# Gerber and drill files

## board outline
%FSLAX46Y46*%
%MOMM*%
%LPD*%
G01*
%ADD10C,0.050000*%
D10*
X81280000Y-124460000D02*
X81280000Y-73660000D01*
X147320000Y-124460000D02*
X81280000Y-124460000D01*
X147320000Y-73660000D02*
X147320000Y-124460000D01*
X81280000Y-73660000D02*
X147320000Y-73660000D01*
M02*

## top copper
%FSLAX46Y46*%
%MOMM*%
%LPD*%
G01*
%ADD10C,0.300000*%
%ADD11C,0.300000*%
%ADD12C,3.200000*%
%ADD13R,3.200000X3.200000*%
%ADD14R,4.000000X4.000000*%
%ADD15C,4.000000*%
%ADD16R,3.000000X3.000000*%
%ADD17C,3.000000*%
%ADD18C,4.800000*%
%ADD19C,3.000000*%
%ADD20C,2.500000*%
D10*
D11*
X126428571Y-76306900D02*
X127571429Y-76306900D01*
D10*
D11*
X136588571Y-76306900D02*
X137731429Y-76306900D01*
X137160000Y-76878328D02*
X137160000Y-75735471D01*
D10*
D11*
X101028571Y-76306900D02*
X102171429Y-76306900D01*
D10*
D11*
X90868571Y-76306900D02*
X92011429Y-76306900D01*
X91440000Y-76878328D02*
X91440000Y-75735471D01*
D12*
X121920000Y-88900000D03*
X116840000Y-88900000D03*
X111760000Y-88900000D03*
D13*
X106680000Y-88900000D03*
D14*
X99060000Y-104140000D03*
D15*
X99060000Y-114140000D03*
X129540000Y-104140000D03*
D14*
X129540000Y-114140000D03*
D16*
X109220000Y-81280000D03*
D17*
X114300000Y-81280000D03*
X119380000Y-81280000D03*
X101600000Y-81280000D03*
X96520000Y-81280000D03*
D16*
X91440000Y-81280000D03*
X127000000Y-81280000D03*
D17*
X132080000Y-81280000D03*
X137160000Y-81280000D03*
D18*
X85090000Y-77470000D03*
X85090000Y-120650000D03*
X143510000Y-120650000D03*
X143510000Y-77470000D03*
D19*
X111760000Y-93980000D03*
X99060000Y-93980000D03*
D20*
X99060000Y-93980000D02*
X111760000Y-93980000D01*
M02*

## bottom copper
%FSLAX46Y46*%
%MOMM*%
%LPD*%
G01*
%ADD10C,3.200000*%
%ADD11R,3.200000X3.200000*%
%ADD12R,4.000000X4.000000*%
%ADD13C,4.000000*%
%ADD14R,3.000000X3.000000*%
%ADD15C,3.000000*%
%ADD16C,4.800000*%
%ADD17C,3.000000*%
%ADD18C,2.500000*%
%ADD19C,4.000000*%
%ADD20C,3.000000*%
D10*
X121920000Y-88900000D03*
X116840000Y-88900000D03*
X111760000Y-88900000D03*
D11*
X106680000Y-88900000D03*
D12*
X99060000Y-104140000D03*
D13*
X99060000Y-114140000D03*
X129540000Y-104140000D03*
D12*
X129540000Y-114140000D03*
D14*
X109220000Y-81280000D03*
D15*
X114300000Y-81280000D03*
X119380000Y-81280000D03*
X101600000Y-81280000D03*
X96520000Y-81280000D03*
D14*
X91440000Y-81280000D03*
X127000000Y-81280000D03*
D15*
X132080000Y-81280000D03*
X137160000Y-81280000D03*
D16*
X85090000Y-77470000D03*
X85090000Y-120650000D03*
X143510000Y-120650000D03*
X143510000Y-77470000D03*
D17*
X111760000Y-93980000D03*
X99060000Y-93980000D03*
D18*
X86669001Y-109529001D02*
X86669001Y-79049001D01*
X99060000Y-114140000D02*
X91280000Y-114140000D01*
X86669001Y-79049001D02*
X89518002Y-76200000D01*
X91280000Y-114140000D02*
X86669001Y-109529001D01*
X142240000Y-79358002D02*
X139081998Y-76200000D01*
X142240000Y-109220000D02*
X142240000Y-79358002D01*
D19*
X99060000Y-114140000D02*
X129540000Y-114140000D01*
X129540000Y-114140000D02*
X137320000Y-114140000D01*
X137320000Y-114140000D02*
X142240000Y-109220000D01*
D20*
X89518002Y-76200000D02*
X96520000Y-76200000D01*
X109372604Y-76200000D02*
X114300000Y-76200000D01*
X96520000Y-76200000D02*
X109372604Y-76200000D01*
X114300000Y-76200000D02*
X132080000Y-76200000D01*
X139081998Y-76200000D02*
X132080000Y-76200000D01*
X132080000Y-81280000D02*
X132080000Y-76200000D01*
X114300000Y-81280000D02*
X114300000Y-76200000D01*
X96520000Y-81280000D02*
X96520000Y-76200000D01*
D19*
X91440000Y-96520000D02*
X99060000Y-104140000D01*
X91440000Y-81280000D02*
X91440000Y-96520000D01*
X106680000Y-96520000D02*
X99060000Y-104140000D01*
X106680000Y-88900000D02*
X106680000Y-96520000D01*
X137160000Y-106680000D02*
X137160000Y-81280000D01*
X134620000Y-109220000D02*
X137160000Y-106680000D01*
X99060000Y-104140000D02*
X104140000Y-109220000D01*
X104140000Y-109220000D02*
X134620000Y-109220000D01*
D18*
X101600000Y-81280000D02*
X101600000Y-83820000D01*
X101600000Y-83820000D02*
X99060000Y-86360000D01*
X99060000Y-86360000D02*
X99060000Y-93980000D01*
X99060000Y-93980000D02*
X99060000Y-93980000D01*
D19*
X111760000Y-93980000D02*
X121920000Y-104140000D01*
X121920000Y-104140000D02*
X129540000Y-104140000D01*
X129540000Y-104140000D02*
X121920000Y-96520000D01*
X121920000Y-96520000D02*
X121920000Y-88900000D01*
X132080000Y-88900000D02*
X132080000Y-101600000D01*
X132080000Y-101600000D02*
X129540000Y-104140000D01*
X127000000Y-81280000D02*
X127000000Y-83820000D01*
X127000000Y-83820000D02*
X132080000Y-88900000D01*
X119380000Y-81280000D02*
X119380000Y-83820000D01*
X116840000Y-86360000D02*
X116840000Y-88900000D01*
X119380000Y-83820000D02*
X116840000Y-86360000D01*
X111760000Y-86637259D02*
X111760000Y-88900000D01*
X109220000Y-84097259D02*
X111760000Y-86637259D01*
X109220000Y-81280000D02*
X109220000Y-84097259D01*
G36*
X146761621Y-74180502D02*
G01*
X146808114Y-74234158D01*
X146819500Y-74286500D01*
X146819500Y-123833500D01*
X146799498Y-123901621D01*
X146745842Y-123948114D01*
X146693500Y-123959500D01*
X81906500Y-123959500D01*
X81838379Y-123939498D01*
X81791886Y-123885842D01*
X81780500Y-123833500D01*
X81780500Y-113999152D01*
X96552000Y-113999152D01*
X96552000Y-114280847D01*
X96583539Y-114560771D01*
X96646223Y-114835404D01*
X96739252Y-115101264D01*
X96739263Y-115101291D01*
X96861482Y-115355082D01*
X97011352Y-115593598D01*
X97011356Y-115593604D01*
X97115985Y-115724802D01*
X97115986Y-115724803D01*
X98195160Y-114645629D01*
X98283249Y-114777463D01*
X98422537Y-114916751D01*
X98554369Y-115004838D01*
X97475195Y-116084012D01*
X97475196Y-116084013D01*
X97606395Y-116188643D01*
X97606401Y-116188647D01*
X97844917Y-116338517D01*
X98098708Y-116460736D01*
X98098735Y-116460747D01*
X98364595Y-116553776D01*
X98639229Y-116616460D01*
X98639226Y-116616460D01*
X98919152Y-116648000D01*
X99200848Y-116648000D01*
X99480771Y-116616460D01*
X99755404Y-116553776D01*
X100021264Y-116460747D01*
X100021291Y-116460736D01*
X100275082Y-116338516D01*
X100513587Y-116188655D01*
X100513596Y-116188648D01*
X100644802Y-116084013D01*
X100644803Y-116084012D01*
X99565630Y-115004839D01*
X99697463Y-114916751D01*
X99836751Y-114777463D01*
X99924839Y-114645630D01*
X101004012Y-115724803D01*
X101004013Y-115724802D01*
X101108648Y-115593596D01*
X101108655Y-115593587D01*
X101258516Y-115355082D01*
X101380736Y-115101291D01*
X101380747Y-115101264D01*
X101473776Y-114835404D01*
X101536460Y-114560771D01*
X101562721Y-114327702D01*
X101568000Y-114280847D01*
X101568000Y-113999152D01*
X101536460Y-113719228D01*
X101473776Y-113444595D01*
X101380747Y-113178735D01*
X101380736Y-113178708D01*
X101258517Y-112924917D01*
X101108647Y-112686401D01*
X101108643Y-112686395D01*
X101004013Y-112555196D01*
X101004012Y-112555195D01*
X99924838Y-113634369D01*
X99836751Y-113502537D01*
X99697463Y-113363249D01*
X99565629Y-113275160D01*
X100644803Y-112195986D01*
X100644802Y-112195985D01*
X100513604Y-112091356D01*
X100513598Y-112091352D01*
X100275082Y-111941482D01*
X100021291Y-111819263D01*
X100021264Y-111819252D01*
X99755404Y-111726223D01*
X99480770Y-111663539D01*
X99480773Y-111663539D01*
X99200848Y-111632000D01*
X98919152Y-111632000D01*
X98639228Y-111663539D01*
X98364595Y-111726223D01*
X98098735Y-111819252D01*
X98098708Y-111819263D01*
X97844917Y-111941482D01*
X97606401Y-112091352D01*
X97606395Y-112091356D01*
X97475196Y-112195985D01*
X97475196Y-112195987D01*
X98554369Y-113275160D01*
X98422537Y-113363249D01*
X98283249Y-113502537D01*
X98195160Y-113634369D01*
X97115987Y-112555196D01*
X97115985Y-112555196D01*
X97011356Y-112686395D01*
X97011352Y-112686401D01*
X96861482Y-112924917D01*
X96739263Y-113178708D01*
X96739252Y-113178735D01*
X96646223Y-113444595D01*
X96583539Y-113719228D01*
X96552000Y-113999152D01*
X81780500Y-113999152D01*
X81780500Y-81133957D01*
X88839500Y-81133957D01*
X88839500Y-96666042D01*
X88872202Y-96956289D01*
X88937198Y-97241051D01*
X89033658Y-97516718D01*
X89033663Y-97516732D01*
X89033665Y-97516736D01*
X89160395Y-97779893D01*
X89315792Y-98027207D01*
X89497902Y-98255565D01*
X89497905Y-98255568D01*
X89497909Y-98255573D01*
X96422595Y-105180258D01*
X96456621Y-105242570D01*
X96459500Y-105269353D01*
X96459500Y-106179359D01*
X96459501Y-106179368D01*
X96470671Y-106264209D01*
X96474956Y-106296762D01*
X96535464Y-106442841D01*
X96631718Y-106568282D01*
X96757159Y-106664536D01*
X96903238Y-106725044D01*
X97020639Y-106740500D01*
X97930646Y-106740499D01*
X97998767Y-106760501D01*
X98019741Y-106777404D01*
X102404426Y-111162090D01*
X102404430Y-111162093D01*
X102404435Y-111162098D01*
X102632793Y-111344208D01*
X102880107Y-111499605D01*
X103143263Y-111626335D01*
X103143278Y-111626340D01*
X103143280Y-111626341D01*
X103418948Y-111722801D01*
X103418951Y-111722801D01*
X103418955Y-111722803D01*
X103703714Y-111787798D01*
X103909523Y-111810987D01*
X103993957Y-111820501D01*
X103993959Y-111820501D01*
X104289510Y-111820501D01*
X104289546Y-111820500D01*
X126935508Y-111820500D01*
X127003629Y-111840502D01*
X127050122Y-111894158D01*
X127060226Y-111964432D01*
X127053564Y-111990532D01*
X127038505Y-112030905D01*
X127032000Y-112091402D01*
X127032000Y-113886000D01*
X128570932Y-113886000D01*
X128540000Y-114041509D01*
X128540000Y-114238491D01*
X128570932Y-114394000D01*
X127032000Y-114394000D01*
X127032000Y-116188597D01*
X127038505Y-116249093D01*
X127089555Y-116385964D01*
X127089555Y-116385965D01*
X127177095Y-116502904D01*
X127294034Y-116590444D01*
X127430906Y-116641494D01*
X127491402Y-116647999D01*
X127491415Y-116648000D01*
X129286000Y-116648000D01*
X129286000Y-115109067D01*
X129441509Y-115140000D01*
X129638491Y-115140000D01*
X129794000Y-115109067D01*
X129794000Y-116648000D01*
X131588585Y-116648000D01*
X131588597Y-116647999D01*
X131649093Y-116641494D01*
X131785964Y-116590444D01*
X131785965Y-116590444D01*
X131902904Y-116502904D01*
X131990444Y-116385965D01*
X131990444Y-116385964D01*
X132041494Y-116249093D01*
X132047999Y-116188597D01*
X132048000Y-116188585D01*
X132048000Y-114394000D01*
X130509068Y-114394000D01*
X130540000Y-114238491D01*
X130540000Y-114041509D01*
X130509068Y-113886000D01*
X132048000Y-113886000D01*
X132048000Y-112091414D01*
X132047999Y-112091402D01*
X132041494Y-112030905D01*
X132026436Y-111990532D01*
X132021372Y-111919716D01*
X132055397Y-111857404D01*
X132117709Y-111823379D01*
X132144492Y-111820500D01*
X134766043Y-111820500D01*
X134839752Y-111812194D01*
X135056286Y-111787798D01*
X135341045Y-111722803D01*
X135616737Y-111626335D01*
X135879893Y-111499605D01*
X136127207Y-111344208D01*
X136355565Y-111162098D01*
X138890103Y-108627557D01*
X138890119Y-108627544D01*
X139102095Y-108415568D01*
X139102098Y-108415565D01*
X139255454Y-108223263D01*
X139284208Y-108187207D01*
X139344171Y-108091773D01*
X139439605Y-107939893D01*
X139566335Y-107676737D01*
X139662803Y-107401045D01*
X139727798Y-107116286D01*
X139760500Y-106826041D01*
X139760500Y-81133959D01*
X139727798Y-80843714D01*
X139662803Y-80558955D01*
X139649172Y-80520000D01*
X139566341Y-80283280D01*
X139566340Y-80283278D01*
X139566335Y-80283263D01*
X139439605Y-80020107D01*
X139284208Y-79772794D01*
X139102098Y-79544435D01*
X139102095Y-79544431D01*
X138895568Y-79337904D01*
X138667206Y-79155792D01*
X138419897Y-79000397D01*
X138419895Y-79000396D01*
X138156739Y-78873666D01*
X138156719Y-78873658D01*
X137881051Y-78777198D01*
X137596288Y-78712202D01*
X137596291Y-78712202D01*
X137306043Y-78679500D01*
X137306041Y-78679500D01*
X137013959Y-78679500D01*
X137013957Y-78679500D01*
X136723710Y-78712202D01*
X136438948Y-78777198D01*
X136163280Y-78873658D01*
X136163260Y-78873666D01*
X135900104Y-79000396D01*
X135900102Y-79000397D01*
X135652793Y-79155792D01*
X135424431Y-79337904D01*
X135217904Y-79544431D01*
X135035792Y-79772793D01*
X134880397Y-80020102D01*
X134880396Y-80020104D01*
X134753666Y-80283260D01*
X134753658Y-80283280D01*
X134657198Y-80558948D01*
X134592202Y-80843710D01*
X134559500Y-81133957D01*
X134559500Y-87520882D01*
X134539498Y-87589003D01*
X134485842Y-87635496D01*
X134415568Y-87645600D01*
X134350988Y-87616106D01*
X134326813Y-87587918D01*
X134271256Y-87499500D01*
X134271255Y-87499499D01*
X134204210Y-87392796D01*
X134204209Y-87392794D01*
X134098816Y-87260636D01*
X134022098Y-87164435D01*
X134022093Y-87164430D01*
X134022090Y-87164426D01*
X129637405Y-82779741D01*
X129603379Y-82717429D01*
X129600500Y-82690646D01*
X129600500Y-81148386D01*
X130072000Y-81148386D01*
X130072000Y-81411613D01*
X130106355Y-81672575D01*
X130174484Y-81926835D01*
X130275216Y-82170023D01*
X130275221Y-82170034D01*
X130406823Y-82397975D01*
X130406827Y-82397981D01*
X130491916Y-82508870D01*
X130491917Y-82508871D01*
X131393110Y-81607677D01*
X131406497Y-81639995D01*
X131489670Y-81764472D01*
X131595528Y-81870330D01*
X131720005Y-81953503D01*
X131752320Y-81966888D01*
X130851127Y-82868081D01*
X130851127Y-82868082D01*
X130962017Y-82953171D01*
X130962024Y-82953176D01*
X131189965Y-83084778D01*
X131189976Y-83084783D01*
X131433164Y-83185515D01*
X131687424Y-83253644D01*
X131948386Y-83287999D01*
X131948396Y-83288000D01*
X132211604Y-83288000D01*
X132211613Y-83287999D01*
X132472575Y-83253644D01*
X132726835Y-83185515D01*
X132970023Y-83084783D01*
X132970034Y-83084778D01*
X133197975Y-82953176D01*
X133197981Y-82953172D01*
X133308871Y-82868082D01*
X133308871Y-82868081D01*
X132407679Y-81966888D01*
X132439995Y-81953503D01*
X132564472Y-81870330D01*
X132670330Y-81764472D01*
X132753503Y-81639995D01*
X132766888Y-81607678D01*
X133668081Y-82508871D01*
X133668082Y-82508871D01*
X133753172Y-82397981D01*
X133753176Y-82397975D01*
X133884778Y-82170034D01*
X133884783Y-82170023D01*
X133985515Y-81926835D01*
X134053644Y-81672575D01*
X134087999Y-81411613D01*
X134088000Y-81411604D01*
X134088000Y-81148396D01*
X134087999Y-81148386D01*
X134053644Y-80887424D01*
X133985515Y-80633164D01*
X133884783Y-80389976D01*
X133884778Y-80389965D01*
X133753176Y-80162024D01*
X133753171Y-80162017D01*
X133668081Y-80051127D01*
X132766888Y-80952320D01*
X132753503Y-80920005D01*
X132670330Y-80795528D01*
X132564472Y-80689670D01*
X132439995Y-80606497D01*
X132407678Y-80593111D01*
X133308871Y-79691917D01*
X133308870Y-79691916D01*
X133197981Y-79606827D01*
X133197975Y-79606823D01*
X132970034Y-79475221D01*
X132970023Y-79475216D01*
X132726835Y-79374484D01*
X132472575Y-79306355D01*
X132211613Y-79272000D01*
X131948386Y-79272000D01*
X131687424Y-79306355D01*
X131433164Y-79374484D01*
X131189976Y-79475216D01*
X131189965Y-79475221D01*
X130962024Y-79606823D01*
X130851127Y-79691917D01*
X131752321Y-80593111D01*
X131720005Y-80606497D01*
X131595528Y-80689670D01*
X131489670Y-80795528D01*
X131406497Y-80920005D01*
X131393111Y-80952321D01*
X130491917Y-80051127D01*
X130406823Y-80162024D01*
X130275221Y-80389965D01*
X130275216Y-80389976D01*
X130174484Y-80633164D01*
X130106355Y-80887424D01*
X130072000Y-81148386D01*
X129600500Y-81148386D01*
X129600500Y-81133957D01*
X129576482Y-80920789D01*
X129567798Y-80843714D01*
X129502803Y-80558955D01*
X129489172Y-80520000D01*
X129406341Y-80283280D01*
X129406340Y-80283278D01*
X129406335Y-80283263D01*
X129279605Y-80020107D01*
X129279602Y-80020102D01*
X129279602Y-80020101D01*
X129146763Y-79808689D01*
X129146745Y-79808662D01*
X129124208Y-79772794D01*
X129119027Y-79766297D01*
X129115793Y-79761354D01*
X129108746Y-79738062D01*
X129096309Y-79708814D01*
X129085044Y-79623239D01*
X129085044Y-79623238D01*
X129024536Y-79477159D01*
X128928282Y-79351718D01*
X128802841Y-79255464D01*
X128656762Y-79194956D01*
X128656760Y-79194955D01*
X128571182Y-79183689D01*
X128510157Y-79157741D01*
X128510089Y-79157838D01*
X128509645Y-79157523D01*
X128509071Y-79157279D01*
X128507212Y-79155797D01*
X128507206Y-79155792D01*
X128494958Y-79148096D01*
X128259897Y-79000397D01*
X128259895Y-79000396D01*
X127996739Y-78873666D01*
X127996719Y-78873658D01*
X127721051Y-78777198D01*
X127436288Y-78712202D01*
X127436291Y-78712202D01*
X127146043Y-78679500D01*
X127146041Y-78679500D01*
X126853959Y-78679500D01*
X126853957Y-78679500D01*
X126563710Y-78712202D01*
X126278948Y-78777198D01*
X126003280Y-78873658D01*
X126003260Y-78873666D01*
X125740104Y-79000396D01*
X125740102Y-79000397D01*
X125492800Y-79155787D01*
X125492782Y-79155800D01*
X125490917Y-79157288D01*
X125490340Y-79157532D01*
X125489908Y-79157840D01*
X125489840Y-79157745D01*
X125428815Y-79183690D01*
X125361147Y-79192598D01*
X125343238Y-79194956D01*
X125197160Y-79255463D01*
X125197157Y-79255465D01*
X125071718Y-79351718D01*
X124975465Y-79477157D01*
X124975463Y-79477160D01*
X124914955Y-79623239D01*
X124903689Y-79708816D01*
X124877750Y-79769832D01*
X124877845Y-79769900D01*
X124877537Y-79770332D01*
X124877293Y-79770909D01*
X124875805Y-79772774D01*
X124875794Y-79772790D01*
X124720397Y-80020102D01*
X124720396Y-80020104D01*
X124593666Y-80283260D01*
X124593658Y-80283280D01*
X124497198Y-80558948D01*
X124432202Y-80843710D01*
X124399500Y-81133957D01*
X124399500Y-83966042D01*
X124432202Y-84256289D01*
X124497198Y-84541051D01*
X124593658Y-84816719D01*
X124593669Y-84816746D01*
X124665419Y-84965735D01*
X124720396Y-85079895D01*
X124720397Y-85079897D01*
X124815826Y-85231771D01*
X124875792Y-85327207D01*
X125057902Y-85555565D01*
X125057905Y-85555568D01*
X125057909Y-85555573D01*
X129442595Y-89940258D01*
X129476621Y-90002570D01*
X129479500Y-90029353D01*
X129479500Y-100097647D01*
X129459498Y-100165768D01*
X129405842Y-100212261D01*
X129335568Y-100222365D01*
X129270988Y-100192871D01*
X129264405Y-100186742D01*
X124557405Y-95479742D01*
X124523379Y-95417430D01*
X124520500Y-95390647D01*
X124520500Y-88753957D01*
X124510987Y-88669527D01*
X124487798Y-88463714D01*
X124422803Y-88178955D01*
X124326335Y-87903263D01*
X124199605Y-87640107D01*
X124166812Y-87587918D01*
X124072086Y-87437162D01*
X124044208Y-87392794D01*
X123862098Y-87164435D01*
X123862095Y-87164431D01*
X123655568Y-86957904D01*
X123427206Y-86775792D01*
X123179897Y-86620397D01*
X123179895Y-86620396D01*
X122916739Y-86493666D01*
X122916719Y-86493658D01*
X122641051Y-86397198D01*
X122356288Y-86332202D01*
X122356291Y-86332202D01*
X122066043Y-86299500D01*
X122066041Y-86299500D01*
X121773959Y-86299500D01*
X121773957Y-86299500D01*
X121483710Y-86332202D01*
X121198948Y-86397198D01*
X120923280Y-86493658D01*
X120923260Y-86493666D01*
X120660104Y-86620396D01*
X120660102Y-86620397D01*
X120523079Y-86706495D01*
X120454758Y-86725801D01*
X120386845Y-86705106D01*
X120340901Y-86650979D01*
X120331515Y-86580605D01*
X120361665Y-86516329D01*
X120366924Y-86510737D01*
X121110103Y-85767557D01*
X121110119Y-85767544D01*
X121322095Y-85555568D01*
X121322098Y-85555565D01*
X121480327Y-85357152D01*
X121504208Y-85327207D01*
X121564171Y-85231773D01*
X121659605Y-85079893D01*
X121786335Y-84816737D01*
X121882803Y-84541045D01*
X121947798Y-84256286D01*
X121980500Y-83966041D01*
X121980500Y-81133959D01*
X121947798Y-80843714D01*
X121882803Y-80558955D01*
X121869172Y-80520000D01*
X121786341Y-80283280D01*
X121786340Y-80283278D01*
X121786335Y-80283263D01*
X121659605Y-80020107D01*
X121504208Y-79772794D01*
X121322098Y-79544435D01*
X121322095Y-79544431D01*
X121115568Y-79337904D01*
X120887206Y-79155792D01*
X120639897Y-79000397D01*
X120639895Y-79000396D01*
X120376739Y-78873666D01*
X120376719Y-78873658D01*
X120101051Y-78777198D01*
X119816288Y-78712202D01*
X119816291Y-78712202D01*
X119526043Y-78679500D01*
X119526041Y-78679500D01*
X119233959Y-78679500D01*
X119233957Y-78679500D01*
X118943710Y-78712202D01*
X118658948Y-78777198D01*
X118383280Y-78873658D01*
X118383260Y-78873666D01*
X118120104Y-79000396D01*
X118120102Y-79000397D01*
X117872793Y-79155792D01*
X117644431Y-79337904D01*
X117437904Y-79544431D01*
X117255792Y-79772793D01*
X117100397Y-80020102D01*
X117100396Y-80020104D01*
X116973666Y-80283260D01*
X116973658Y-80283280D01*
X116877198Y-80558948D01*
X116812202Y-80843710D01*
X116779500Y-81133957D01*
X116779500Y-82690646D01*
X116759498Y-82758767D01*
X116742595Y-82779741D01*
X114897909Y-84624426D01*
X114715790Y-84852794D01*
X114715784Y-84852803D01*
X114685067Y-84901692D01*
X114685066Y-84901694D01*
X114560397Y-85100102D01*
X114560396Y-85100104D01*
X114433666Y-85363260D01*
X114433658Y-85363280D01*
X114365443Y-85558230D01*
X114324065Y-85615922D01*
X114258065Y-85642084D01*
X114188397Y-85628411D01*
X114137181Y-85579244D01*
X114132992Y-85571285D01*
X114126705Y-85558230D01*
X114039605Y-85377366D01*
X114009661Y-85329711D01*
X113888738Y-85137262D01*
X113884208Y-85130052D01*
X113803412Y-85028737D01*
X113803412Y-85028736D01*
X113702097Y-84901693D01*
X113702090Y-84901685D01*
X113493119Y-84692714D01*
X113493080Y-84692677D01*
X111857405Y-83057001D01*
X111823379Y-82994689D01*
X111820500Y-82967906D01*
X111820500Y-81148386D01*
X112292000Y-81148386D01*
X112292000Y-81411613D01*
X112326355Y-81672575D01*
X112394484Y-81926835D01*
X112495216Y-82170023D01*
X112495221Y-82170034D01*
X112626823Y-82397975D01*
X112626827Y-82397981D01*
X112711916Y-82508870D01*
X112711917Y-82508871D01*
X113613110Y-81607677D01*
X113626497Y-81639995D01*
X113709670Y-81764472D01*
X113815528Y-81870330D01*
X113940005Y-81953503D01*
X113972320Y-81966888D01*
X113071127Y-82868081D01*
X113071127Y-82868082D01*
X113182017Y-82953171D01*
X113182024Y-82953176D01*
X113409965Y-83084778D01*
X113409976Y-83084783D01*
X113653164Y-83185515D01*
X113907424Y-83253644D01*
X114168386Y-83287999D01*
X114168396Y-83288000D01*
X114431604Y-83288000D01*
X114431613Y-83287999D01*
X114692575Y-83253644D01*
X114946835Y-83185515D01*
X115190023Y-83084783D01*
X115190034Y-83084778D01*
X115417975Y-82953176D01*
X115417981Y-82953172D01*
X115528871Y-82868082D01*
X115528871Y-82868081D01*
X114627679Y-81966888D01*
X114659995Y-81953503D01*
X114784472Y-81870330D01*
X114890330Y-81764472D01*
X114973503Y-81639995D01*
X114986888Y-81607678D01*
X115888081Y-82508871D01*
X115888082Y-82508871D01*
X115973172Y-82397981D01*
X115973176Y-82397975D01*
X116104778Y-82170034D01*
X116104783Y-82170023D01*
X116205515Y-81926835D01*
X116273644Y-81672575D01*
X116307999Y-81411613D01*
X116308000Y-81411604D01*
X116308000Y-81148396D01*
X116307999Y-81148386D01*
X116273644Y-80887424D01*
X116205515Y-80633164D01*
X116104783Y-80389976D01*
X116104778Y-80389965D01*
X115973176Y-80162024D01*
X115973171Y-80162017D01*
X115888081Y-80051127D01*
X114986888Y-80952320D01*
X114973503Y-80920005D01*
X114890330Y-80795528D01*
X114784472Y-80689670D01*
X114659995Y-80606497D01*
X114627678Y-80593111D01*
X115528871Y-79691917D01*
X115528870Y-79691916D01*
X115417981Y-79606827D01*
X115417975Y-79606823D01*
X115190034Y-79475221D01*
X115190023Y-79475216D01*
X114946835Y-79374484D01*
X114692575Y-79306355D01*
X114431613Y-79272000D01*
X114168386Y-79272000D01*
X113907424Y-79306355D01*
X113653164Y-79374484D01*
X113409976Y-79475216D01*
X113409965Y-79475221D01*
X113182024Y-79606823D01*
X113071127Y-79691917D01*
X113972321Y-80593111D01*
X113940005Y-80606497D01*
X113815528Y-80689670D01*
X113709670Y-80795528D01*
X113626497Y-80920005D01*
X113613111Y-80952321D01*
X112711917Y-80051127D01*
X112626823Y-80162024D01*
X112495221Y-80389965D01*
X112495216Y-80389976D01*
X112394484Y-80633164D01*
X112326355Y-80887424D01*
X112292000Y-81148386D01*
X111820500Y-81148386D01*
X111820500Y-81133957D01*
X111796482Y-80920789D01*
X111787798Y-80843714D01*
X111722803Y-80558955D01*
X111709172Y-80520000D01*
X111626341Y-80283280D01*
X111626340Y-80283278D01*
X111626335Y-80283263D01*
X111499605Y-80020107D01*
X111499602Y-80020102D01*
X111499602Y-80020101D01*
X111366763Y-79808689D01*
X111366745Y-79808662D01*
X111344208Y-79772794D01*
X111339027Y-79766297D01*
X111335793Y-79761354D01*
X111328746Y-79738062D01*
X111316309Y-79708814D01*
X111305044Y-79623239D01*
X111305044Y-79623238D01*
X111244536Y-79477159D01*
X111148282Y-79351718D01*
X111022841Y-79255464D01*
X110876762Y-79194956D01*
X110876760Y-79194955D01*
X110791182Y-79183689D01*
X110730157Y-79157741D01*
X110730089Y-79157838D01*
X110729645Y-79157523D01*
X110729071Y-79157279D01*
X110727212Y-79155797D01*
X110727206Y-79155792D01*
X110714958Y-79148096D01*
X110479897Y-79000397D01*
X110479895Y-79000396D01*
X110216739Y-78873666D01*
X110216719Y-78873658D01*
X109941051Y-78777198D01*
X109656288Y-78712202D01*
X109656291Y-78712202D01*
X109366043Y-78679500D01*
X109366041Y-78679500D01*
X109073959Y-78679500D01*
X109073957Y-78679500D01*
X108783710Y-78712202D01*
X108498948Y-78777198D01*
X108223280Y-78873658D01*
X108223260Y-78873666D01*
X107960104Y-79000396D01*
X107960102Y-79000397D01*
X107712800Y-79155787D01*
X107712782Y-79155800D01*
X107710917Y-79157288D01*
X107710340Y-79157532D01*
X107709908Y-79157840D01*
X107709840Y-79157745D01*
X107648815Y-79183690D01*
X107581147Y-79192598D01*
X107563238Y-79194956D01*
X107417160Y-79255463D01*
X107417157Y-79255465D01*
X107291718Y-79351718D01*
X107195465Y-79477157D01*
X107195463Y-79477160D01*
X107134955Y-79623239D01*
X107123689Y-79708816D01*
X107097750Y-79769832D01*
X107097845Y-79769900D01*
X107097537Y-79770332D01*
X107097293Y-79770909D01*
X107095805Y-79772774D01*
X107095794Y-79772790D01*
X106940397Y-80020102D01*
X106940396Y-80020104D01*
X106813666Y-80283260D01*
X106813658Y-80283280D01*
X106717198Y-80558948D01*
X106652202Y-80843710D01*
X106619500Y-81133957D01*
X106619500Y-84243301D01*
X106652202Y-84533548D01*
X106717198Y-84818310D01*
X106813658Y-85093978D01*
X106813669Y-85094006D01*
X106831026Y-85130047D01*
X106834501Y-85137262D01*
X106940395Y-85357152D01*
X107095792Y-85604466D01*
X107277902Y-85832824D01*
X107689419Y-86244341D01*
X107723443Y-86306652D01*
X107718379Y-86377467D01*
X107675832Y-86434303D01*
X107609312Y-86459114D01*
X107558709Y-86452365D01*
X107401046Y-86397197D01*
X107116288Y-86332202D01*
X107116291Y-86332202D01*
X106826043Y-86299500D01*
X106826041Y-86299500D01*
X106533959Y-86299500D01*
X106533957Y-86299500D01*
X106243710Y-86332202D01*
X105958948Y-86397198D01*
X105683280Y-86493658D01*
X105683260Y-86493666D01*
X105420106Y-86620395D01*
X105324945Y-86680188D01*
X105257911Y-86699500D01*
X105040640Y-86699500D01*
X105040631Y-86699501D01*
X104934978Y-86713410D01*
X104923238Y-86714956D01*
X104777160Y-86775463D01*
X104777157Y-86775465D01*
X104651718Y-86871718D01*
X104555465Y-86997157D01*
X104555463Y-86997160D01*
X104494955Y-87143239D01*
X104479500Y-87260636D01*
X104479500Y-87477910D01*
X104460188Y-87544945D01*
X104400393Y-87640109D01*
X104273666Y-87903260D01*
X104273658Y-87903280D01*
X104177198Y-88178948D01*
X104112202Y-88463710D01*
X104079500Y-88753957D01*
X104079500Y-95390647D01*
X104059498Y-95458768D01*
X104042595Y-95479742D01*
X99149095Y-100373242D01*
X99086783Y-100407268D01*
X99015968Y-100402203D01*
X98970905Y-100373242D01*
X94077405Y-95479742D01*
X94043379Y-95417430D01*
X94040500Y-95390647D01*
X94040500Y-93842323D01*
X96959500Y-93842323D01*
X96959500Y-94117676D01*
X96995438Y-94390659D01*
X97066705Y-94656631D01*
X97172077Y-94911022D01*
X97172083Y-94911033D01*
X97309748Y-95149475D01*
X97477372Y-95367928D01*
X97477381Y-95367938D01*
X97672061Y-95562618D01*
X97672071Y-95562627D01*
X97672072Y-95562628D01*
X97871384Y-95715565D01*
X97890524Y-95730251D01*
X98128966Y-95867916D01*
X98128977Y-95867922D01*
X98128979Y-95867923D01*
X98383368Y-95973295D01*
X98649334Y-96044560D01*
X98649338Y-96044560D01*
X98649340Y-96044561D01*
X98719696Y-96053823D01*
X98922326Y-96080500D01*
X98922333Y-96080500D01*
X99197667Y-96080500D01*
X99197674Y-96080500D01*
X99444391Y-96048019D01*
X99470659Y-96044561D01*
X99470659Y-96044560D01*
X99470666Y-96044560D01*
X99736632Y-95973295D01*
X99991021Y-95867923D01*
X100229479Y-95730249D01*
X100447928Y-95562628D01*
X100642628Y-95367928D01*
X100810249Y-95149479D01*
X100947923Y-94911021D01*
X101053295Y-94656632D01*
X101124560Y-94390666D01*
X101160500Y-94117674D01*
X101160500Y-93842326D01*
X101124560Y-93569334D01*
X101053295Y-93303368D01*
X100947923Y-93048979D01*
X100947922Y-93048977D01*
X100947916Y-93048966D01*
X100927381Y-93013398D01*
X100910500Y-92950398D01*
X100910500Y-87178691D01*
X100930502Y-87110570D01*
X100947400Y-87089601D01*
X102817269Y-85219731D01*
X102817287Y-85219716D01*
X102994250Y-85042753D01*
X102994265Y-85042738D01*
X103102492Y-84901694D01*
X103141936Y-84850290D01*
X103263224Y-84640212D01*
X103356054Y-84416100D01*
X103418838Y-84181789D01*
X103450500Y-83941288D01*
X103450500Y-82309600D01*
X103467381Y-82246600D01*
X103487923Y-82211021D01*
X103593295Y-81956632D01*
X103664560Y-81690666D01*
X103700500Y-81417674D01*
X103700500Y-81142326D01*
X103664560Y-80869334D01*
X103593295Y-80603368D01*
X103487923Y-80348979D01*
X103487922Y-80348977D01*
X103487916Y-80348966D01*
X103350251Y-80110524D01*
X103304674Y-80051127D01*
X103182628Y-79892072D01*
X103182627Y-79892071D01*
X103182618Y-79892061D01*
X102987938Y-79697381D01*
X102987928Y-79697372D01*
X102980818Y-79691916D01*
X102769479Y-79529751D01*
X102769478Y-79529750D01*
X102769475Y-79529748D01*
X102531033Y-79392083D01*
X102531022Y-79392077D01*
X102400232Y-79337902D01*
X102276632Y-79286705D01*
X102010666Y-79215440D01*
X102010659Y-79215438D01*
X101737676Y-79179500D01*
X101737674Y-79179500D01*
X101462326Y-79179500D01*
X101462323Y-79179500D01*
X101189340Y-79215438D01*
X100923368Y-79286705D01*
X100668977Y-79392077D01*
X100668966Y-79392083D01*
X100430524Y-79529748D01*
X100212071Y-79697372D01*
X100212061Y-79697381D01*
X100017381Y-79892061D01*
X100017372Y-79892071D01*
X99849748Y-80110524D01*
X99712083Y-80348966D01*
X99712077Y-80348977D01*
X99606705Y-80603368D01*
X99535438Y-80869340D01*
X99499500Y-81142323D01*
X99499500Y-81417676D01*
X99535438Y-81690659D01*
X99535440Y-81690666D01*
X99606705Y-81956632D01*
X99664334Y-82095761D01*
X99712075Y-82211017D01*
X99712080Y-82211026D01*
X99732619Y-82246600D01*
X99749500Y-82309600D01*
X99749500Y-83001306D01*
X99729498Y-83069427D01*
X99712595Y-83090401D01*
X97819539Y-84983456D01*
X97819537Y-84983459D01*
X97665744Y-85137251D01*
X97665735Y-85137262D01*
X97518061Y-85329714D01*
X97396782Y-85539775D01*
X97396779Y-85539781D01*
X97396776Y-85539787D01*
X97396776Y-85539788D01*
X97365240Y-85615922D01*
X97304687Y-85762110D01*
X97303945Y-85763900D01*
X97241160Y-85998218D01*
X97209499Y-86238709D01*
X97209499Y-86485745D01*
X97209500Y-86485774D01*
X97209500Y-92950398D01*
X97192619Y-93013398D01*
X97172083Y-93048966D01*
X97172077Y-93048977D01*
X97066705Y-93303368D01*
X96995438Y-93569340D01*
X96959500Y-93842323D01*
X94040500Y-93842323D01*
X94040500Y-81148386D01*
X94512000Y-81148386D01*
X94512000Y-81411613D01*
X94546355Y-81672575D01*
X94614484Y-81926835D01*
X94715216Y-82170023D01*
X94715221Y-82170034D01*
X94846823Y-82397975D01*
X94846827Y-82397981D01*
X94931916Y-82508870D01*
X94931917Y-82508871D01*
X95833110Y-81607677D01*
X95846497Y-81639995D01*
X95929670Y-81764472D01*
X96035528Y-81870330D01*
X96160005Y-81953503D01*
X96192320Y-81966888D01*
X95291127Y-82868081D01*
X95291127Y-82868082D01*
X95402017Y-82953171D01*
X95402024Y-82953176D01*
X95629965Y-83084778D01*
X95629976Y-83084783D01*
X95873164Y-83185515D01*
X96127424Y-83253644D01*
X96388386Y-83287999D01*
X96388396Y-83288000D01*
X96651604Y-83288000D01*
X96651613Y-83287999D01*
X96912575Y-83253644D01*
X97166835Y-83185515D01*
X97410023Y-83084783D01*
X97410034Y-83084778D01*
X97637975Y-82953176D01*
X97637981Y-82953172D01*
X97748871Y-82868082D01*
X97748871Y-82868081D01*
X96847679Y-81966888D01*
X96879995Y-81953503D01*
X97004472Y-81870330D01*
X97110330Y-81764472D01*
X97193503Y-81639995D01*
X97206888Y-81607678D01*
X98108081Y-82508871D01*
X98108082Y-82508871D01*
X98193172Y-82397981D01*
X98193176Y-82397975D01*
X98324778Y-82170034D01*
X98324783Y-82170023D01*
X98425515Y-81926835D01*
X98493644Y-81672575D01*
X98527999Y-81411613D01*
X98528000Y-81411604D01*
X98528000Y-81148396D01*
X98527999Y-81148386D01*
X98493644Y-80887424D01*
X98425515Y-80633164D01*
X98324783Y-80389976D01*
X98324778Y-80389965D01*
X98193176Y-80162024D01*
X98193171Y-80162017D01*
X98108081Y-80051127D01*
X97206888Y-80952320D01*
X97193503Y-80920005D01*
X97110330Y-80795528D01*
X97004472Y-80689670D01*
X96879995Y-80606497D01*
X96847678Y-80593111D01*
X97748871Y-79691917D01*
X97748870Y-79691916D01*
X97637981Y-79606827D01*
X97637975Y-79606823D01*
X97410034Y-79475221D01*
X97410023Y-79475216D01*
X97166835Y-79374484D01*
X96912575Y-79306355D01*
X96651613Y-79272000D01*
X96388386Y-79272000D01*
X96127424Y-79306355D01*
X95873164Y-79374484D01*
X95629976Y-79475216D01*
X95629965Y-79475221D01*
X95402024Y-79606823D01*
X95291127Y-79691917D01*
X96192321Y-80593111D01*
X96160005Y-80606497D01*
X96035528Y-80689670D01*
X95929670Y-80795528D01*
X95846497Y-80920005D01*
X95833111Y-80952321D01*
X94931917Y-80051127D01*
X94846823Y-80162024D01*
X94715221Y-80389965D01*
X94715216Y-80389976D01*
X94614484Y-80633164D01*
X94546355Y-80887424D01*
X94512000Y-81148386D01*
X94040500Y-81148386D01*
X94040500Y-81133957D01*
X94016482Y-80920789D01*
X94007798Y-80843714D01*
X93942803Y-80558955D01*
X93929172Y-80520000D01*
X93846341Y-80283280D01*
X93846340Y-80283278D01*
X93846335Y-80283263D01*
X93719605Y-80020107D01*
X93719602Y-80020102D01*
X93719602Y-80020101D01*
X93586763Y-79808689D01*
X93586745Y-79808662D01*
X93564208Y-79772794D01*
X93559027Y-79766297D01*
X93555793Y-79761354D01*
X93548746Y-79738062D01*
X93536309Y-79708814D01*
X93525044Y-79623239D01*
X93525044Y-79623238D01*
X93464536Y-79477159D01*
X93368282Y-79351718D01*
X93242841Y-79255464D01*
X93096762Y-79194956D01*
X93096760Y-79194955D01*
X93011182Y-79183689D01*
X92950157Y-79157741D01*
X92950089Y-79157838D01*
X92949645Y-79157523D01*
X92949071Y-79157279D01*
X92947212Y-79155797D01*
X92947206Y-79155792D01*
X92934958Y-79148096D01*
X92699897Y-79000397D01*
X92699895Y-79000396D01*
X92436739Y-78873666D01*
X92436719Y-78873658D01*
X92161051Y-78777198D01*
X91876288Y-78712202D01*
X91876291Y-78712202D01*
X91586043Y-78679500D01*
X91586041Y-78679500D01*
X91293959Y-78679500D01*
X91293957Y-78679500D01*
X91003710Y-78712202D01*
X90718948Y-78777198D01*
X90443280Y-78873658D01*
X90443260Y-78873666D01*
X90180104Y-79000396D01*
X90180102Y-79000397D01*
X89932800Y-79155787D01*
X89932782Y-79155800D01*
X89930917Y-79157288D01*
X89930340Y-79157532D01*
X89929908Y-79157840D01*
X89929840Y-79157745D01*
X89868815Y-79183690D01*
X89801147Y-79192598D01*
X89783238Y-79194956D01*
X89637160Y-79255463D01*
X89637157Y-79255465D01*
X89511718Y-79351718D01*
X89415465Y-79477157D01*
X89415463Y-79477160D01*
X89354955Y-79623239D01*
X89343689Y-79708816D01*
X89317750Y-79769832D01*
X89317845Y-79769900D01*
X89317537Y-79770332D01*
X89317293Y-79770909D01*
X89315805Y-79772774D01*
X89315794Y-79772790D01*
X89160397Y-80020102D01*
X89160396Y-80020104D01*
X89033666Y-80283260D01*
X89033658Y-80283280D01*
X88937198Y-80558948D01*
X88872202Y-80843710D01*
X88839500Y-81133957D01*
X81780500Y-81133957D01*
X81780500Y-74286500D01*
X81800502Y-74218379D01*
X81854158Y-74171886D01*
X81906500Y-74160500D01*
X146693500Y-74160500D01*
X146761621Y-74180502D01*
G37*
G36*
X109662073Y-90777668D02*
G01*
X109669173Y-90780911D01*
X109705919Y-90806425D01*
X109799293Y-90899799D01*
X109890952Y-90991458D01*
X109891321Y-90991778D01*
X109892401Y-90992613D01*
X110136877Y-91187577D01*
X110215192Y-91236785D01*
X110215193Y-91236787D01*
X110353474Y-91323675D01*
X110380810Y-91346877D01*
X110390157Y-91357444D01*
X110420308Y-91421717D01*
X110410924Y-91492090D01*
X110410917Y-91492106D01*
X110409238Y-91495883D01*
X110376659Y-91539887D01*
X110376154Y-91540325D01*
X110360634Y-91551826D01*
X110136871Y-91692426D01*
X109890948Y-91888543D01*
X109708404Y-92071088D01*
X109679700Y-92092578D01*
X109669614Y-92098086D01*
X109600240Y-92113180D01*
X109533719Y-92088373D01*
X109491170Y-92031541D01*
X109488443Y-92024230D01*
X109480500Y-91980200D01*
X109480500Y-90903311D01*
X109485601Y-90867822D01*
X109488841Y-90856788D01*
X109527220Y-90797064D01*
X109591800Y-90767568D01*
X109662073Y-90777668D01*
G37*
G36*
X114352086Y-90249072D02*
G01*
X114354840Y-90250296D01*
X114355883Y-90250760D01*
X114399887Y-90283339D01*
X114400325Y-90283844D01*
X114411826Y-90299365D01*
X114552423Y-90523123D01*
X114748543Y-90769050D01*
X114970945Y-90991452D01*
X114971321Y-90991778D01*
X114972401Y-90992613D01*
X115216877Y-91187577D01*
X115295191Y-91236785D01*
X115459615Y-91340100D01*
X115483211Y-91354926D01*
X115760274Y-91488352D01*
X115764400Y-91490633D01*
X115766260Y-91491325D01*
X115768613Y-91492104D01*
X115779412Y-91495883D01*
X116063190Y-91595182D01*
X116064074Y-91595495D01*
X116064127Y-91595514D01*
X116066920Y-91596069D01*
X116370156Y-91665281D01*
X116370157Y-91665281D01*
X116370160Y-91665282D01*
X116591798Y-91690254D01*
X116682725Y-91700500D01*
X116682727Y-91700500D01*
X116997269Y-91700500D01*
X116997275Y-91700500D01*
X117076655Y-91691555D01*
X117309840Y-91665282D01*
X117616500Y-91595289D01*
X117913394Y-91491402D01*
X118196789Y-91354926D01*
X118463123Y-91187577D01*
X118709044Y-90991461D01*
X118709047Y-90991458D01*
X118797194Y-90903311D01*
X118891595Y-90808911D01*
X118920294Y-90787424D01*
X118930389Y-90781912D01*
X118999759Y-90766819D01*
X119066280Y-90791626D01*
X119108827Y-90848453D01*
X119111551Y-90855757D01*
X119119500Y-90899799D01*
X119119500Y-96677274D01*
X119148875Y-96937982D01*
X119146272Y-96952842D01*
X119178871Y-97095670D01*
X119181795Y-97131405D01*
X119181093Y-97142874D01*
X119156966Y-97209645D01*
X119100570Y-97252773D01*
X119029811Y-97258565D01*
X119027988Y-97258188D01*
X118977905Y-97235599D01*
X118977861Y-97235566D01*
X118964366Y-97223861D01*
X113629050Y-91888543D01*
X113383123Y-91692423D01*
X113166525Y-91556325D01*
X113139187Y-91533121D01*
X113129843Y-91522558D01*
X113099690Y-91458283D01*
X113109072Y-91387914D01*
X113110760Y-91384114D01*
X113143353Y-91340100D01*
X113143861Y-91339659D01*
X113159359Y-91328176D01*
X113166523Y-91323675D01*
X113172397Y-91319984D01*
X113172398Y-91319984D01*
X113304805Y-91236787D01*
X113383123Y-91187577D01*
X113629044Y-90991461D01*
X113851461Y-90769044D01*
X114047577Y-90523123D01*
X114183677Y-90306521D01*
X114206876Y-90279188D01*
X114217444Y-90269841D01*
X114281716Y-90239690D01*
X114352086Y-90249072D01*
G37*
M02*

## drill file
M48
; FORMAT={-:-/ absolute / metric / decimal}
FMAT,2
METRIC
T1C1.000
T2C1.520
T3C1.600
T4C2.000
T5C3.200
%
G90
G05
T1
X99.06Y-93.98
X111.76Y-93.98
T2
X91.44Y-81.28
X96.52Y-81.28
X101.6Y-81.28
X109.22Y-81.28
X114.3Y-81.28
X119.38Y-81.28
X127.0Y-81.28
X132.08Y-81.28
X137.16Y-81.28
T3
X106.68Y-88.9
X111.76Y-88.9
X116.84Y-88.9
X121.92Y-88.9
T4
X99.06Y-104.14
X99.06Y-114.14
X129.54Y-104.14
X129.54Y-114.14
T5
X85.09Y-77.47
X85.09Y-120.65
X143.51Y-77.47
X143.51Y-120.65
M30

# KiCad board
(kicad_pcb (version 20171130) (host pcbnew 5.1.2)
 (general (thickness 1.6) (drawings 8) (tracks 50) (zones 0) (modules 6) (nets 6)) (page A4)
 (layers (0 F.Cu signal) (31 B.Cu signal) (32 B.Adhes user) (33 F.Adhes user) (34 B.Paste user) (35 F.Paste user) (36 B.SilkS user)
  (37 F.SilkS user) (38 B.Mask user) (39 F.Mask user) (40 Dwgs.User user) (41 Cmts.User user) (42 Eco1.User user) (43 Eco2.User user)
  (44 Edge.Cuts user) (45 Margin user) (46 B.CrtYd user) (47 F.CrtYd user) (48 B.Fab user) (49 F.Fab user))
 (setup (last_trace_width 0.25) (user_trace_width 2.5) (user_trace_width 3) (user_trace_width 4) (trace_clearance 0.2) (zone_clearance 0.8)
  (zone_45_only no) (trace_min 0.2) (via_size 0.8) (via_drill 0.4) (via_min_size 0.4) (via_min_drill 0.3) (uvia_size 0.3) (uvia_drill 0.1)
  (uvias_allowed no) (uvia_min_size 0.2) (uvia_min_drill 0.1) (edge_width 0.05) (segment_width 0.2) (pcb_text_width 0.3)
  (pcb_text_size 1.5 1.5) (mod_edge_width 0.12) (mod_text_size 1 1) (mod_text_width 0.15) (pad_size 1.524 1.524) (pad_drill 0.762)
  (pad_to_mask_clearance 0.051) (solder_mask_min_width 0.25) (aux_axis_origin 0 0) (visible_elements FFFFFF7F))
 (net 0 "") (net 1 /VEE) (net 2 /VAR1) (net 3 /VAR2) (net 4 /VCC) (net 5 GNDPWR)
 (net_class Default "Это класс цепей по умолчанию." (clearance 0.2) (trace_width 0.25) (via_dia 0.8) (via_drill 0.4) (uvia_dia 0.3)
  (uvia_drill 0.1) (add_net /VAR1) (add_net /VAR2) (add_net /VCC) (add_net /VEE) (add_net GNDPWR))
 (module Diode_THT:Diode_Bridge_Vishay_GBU (layer F.Cu) (at 106.68 88.9)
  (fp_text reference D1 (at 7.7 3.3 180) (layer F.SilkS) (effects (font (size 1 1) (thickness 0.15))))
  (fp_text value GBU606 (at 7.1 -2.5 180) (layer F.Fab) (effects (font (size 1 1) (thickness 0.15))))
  (pad 4 thru_hole circle (at 15.24 0) (size 3.2 3.2) (drill 1.6) (layers *.Cu *.Mask) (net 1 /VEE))
  (pad 3 thru_hole circle (at 10.16 0) (size 3.2 3.2) (drill 1.6) (layers *.Cu *.Mask) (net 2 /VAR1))
  (pad 2 thru_hole circle (at 5.08 0) (size 3.2 3.2) (drill 1.6) (layers *.Cu *.Mask) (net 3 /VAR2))
  (pad 1 thru_hole rect (at 0 0) (size 3.2 3.2) (drill 1.6) (layers *.Cu *.Mask) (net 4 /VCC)))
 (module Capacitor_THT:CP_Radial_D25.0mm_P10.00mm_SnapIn (layer F.Cu) (at 99.06 104.14 270)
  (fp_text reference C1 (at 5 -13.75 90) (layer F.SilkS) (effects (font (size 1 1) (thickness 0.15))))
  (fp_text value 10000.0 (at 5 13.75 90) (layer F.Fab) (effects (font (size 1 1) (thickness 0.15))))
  (pad 1 thru_hole rect (at 0 0 270) (size 4 4) (drill 2) (layers *.Cu *.Mask) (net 4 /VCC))
  (pad 2 thru_hole circle (at 10 0 270) (size 4 4) (drill 2) (layers *.Cu *.Mask) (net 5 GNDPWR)))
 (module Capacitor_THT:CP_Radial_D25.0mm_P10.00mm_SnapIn (layer F.Cu) (at 129.54 114.14 90)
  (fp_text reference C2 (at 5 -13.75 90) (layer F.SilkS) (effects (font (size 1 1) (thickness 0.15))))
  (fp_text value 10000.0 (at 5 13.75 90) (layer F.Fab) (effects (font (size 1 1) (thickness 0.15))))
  (pad 2 thru_hole circle (at 10 0 90) (size 4 4) (drill 2) (layers *.Cu *.Mask) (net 1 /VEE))
  (pad 1 thru_hole rect (at 0 0 90) (size 4 4) (drill 2) (layers *.Cu *.Mask) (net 5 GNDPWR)))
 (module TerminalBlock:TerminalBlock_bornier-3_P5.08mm (layer F.Cu) (at 109.22 81.28)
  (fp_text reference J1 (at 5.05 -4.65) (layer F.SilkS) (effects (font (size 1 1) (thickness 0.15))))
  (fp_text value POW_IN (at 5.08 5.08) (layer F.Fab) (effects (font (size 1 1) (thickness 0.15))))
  (pad 1 thru_hole rect (at 0 0) (size 3 3) (drill 1.52) (layers *.Cu *.Mask) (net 3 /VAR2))
  (pad 2 thru_hole circle (at 5.08 0) (size 3 3) (drill 1.52) (layers *.Cu *.Mask) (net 5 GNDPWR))
  (pad 3 thru_hole circle (at 10.16 0) (size 3 3) (drill 1.52) (layers *.Cu *.Mask) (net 2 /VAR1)))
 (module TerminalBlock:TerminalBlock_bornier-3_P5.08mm (layer F.Cu) (at 91.44 81.28)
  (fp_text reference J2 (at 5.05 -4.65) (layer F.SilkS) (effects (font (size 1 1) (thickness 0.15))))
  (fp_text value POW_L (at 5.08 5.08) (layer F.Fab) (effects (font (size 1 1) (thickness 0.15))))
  (pad 3 thru_hole circle (at 10.16 0) (size 3 3) (drill 1.52) (layers *.Cu *.Mask) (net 1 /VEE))
  (pad 2 thru_hole circle (at 5.08 0) (size 3 3) (drill 1.52) (layers *.Cu *.Mask) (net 5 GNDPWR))
  (pad 1 thru_hole rect (at 0 0) (size 3 3) (drill 1.52) (layers *.Cu *.Mask) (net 4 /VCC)))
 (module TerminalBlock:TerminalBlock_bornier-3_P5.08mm (layer F.Cu) (at 127 81.28)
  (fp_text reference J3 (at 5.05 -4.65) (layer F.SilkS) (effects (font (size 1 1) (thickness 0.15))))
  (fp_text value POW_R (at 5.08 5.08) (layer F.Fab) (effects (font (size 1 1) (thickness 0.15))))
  (pad 1 thru_hole rect (at 0 0) (size 3 3) (drill 1.52) (layers *.Cu *.Mask) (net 1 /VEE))
  (pad 2 thru_hole circle (at 5.08 0) (size 3 3) (drill 1.52) (layers *.Cu *.Mask) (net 5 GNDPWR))
  (pad 3 thru_hole circle (at 10.16 0) (size 3 3) (drill 1.52) (layers *.Cu *.Mask) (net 4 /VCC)))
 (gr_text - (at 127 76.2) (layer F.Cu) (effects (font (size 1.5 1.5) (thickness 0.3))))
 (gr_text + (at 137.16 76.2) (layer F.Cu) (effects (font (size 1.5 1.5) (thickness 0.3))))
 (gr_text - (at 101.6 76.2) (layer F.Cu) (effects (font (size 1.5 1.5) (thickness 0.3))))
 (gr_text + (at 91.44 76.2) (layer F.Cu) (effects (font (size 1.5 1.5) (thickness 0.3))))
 (gr_line (start 81.28 124.46) (end 81.28 73.66) (layer Edge.Cuts) (width 0.05))
 (gr_line (start 147.32 124.46) (end 81.28 124.46) (layer Edge.Cuts) (width 0.05))
 (gr_line (start 147.32 73.66) (end 147.32 124.46) (layer Edge.Cuts) (width 0.05))
 (gr_line (start 81.28 73.66) (end 147.32 73.66) (layer Edge.Cuts) (width 0.05))
 (via (at 85.09 77.47) (size 4.8) (drill 3.2) (layers F.Cu B.Cu) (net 5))
 (via (at 85.09 120.65) (size 4.8) (drill 3.2) (layers F.Cu B.Cu) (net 5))
 (via (at 143.51 120.65) (size 4.8) (drill 3.2) (layers F.Cu B.Cu) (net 5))
 (via (at 143.51 77.47) (size 4.8) (drill 3.2) (layers F.Cu B.Cu) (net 5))
 (segment (start 86.669001 109.529001) (end 86.669001 79.049001) (width 2.5) (layer B.Cu) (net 5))
 (segment (start 99.06 114.14) (end 91.28 114.14) (width 2.5) (layer B.Cu) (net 5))
 (segment (start 86.669001 79.049001) (end 89.518002 76.2) (width 2.5) (layer B.Cu) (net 5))
 (segment (start 91.28 114.14) (end 86.669001 109.529001) (width 2.5) (layer B.Cu) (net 5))
 (segment (start 142.24 79.358002) (end 139.081998 76.2) (width 2.5) (layer B.Cu) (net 5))
 (segment (start 142.24 109.22) (end 142.24 79.358002) (width 2.5) (layer B.Cu) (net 5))
 (segment (start 99.06 114.14) (end 129.54 114.14) (width 4) (layer B.Cu) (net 5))
 (segment (start 129.54 114.14) (end 137.32 114.14) (width 4) (layer B.Cu) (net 5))
 (segment (start 137.32 114.14) (end 142.24 109.22) (width 4) (layer B.Cu) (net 5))
 (segment (start 89.518002 76.2) (end 96.52 76.2) (width 3) (layer B.Cu) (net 5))
 (segment (start 109.372604 76.2) (end 114.3 76.2) (width 3) (layer B.Cu) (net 5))
 (segment (start 96.52 76.2) (end 109.372604 76.2) (width 3) (layer B.Cu) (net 5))
 (segment (start 114.3 76.2) (end 132.08 76.2) (width 3) (layer B.Cu) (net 5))
 (segment (start 139.081998 76.2) (end 132.08 76.2) (width 3) (layer B.Cu) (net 5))
 (segment (start 132.08 81.28) (end 132.08 76.2) (width 3) (layer B.Cu) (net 5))
 (segment (start 114.3 81.28) (end 114.3 76.2) (width 3) (layer B.Cu) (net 5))
 (segment (start 96.52 81.28) (end 96.52 76.2) (width 3) (layer B.Cu) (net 5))
 (segment (start 91.44 96.52) (end 99.06 104.14) (width 4) (layer B.Cu) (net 4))
 (segment (start 91.44 81.28) (end 91.44 96.52) (width 4) (layer B.Cu) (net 4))
 (segment (start 106.68 96.52) (end 99.06 104.14) (width 4) (layer B.Cu) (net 4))
 (segment (start 106.68 88.9) (end 106.68 96.52) (width 4) (layer B.Cu) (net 4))
 (segment (start 137.16 106.68) (end 137.16 81.28) (width 4) (layer B.Cu) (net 4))
 (segment (start 134.62 109.22) (end 137.16 106.68) (width 4) (layer B.Cu) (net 4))
 (segment (start 99.06 104.14) (end 104.14 109.22) (width 4) (layer B.Cu) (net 4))
 (segment (start 104.14 109.22) (end 134.62 109.22) (width 4) (layer B.Cu) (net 4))
 (via (at 111.76 93.98) (size 3) (drill 1) (layers F.Cu B.Cu) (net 1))
 (segment (start 101.6 81.28) (end 101.6 83.82) (width 2.5) (layer B.Cu) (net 1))
 (segment (start 101.6 83.82) (end 99.06 86.36) (width 2.5) (layer B.Cu) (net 1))
 (segment (start 99.06 86.36) (end 99.06 93.98) (width 2.5) (layer B.Cu) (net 1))
 (segment (start 99.06 93.98) (end 99.06 93.98) (width 2.5) (layer B.Cu) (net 1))
 (via (at 99.06 93.98) (size 3) (drill 1) (layers F.Cu B.Cu) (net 1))
 (segment (start 99.06 93.98) (end 111.76 93.98) (width 2.5) (layer F.Cu) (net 1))
 (segment (start 111.76 93.98) (end 121.92 104.14) (width 4) (layer B.Cu) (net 1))
 (segment (start 121.92 104.14) (end 129.54 104.14) (width 4) (layer B.Cu) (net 1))
 (segment (start 129.54 104.14) (end 121.92 96.52) (width 4) (layer B.Cu) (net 1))
 (segment (start 121.92 96.52) (end 121.92 88.9) (width 4) (layer B.Cu) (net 1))
 (segment (start 132.08 88.9) (end 132.08 101.6) (width 4) (layer B.Cu) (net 1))
 (segment (start 132.08 101.6) (end 129.54 104.14) (width 4) (layer B.Cu) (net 1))
 (segment (start 127 81.28) (end 127 83.82) (width 4) (layer B.Cu) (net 1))
 (segment (start 127 83.82) (end 132.08 88.9) (width 4) (layer B.Cu) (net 1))
 (segment (start 119.38 81.28) (end 119.38 83.82) (width 4) (layer B.Cu) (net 2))
 (segment (start 116.84 86.36) (end 116.84 88.9) (width 4) (layer B.Cu) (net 2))
 (segment (start 119.38 83.82) (end 116.84 86.36) (width 4) (layer B.Cu) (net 2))
 (segment (start 111.76 86.637259) (end 111.76 88.9) (width 4) (layer B.Cu) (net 3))
 (segment (start 109.22 84.097259) (end 111.76 86.637259) (width 4) (layer B.Cu) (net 3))
 (segment (start 109.22 81.28) (end 109.22 84.097259) (width 4) (layer B.Cu) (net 3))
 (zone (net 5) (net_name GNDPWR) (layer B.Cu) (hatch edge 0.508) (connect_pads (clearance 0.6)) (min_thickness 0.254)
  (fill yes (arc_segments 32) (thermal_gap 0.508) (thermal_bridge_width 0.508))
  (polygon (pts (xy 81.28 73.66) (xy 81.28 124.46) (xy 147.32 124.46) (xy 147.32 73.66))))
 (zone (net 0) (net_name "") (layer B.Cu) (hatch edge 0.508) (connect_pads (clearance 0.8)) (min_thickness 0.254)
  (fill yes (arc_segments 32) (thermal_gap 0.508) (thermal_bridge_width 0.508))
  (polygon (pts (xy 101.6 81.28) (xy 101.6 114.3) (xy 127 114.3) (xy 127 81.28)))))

